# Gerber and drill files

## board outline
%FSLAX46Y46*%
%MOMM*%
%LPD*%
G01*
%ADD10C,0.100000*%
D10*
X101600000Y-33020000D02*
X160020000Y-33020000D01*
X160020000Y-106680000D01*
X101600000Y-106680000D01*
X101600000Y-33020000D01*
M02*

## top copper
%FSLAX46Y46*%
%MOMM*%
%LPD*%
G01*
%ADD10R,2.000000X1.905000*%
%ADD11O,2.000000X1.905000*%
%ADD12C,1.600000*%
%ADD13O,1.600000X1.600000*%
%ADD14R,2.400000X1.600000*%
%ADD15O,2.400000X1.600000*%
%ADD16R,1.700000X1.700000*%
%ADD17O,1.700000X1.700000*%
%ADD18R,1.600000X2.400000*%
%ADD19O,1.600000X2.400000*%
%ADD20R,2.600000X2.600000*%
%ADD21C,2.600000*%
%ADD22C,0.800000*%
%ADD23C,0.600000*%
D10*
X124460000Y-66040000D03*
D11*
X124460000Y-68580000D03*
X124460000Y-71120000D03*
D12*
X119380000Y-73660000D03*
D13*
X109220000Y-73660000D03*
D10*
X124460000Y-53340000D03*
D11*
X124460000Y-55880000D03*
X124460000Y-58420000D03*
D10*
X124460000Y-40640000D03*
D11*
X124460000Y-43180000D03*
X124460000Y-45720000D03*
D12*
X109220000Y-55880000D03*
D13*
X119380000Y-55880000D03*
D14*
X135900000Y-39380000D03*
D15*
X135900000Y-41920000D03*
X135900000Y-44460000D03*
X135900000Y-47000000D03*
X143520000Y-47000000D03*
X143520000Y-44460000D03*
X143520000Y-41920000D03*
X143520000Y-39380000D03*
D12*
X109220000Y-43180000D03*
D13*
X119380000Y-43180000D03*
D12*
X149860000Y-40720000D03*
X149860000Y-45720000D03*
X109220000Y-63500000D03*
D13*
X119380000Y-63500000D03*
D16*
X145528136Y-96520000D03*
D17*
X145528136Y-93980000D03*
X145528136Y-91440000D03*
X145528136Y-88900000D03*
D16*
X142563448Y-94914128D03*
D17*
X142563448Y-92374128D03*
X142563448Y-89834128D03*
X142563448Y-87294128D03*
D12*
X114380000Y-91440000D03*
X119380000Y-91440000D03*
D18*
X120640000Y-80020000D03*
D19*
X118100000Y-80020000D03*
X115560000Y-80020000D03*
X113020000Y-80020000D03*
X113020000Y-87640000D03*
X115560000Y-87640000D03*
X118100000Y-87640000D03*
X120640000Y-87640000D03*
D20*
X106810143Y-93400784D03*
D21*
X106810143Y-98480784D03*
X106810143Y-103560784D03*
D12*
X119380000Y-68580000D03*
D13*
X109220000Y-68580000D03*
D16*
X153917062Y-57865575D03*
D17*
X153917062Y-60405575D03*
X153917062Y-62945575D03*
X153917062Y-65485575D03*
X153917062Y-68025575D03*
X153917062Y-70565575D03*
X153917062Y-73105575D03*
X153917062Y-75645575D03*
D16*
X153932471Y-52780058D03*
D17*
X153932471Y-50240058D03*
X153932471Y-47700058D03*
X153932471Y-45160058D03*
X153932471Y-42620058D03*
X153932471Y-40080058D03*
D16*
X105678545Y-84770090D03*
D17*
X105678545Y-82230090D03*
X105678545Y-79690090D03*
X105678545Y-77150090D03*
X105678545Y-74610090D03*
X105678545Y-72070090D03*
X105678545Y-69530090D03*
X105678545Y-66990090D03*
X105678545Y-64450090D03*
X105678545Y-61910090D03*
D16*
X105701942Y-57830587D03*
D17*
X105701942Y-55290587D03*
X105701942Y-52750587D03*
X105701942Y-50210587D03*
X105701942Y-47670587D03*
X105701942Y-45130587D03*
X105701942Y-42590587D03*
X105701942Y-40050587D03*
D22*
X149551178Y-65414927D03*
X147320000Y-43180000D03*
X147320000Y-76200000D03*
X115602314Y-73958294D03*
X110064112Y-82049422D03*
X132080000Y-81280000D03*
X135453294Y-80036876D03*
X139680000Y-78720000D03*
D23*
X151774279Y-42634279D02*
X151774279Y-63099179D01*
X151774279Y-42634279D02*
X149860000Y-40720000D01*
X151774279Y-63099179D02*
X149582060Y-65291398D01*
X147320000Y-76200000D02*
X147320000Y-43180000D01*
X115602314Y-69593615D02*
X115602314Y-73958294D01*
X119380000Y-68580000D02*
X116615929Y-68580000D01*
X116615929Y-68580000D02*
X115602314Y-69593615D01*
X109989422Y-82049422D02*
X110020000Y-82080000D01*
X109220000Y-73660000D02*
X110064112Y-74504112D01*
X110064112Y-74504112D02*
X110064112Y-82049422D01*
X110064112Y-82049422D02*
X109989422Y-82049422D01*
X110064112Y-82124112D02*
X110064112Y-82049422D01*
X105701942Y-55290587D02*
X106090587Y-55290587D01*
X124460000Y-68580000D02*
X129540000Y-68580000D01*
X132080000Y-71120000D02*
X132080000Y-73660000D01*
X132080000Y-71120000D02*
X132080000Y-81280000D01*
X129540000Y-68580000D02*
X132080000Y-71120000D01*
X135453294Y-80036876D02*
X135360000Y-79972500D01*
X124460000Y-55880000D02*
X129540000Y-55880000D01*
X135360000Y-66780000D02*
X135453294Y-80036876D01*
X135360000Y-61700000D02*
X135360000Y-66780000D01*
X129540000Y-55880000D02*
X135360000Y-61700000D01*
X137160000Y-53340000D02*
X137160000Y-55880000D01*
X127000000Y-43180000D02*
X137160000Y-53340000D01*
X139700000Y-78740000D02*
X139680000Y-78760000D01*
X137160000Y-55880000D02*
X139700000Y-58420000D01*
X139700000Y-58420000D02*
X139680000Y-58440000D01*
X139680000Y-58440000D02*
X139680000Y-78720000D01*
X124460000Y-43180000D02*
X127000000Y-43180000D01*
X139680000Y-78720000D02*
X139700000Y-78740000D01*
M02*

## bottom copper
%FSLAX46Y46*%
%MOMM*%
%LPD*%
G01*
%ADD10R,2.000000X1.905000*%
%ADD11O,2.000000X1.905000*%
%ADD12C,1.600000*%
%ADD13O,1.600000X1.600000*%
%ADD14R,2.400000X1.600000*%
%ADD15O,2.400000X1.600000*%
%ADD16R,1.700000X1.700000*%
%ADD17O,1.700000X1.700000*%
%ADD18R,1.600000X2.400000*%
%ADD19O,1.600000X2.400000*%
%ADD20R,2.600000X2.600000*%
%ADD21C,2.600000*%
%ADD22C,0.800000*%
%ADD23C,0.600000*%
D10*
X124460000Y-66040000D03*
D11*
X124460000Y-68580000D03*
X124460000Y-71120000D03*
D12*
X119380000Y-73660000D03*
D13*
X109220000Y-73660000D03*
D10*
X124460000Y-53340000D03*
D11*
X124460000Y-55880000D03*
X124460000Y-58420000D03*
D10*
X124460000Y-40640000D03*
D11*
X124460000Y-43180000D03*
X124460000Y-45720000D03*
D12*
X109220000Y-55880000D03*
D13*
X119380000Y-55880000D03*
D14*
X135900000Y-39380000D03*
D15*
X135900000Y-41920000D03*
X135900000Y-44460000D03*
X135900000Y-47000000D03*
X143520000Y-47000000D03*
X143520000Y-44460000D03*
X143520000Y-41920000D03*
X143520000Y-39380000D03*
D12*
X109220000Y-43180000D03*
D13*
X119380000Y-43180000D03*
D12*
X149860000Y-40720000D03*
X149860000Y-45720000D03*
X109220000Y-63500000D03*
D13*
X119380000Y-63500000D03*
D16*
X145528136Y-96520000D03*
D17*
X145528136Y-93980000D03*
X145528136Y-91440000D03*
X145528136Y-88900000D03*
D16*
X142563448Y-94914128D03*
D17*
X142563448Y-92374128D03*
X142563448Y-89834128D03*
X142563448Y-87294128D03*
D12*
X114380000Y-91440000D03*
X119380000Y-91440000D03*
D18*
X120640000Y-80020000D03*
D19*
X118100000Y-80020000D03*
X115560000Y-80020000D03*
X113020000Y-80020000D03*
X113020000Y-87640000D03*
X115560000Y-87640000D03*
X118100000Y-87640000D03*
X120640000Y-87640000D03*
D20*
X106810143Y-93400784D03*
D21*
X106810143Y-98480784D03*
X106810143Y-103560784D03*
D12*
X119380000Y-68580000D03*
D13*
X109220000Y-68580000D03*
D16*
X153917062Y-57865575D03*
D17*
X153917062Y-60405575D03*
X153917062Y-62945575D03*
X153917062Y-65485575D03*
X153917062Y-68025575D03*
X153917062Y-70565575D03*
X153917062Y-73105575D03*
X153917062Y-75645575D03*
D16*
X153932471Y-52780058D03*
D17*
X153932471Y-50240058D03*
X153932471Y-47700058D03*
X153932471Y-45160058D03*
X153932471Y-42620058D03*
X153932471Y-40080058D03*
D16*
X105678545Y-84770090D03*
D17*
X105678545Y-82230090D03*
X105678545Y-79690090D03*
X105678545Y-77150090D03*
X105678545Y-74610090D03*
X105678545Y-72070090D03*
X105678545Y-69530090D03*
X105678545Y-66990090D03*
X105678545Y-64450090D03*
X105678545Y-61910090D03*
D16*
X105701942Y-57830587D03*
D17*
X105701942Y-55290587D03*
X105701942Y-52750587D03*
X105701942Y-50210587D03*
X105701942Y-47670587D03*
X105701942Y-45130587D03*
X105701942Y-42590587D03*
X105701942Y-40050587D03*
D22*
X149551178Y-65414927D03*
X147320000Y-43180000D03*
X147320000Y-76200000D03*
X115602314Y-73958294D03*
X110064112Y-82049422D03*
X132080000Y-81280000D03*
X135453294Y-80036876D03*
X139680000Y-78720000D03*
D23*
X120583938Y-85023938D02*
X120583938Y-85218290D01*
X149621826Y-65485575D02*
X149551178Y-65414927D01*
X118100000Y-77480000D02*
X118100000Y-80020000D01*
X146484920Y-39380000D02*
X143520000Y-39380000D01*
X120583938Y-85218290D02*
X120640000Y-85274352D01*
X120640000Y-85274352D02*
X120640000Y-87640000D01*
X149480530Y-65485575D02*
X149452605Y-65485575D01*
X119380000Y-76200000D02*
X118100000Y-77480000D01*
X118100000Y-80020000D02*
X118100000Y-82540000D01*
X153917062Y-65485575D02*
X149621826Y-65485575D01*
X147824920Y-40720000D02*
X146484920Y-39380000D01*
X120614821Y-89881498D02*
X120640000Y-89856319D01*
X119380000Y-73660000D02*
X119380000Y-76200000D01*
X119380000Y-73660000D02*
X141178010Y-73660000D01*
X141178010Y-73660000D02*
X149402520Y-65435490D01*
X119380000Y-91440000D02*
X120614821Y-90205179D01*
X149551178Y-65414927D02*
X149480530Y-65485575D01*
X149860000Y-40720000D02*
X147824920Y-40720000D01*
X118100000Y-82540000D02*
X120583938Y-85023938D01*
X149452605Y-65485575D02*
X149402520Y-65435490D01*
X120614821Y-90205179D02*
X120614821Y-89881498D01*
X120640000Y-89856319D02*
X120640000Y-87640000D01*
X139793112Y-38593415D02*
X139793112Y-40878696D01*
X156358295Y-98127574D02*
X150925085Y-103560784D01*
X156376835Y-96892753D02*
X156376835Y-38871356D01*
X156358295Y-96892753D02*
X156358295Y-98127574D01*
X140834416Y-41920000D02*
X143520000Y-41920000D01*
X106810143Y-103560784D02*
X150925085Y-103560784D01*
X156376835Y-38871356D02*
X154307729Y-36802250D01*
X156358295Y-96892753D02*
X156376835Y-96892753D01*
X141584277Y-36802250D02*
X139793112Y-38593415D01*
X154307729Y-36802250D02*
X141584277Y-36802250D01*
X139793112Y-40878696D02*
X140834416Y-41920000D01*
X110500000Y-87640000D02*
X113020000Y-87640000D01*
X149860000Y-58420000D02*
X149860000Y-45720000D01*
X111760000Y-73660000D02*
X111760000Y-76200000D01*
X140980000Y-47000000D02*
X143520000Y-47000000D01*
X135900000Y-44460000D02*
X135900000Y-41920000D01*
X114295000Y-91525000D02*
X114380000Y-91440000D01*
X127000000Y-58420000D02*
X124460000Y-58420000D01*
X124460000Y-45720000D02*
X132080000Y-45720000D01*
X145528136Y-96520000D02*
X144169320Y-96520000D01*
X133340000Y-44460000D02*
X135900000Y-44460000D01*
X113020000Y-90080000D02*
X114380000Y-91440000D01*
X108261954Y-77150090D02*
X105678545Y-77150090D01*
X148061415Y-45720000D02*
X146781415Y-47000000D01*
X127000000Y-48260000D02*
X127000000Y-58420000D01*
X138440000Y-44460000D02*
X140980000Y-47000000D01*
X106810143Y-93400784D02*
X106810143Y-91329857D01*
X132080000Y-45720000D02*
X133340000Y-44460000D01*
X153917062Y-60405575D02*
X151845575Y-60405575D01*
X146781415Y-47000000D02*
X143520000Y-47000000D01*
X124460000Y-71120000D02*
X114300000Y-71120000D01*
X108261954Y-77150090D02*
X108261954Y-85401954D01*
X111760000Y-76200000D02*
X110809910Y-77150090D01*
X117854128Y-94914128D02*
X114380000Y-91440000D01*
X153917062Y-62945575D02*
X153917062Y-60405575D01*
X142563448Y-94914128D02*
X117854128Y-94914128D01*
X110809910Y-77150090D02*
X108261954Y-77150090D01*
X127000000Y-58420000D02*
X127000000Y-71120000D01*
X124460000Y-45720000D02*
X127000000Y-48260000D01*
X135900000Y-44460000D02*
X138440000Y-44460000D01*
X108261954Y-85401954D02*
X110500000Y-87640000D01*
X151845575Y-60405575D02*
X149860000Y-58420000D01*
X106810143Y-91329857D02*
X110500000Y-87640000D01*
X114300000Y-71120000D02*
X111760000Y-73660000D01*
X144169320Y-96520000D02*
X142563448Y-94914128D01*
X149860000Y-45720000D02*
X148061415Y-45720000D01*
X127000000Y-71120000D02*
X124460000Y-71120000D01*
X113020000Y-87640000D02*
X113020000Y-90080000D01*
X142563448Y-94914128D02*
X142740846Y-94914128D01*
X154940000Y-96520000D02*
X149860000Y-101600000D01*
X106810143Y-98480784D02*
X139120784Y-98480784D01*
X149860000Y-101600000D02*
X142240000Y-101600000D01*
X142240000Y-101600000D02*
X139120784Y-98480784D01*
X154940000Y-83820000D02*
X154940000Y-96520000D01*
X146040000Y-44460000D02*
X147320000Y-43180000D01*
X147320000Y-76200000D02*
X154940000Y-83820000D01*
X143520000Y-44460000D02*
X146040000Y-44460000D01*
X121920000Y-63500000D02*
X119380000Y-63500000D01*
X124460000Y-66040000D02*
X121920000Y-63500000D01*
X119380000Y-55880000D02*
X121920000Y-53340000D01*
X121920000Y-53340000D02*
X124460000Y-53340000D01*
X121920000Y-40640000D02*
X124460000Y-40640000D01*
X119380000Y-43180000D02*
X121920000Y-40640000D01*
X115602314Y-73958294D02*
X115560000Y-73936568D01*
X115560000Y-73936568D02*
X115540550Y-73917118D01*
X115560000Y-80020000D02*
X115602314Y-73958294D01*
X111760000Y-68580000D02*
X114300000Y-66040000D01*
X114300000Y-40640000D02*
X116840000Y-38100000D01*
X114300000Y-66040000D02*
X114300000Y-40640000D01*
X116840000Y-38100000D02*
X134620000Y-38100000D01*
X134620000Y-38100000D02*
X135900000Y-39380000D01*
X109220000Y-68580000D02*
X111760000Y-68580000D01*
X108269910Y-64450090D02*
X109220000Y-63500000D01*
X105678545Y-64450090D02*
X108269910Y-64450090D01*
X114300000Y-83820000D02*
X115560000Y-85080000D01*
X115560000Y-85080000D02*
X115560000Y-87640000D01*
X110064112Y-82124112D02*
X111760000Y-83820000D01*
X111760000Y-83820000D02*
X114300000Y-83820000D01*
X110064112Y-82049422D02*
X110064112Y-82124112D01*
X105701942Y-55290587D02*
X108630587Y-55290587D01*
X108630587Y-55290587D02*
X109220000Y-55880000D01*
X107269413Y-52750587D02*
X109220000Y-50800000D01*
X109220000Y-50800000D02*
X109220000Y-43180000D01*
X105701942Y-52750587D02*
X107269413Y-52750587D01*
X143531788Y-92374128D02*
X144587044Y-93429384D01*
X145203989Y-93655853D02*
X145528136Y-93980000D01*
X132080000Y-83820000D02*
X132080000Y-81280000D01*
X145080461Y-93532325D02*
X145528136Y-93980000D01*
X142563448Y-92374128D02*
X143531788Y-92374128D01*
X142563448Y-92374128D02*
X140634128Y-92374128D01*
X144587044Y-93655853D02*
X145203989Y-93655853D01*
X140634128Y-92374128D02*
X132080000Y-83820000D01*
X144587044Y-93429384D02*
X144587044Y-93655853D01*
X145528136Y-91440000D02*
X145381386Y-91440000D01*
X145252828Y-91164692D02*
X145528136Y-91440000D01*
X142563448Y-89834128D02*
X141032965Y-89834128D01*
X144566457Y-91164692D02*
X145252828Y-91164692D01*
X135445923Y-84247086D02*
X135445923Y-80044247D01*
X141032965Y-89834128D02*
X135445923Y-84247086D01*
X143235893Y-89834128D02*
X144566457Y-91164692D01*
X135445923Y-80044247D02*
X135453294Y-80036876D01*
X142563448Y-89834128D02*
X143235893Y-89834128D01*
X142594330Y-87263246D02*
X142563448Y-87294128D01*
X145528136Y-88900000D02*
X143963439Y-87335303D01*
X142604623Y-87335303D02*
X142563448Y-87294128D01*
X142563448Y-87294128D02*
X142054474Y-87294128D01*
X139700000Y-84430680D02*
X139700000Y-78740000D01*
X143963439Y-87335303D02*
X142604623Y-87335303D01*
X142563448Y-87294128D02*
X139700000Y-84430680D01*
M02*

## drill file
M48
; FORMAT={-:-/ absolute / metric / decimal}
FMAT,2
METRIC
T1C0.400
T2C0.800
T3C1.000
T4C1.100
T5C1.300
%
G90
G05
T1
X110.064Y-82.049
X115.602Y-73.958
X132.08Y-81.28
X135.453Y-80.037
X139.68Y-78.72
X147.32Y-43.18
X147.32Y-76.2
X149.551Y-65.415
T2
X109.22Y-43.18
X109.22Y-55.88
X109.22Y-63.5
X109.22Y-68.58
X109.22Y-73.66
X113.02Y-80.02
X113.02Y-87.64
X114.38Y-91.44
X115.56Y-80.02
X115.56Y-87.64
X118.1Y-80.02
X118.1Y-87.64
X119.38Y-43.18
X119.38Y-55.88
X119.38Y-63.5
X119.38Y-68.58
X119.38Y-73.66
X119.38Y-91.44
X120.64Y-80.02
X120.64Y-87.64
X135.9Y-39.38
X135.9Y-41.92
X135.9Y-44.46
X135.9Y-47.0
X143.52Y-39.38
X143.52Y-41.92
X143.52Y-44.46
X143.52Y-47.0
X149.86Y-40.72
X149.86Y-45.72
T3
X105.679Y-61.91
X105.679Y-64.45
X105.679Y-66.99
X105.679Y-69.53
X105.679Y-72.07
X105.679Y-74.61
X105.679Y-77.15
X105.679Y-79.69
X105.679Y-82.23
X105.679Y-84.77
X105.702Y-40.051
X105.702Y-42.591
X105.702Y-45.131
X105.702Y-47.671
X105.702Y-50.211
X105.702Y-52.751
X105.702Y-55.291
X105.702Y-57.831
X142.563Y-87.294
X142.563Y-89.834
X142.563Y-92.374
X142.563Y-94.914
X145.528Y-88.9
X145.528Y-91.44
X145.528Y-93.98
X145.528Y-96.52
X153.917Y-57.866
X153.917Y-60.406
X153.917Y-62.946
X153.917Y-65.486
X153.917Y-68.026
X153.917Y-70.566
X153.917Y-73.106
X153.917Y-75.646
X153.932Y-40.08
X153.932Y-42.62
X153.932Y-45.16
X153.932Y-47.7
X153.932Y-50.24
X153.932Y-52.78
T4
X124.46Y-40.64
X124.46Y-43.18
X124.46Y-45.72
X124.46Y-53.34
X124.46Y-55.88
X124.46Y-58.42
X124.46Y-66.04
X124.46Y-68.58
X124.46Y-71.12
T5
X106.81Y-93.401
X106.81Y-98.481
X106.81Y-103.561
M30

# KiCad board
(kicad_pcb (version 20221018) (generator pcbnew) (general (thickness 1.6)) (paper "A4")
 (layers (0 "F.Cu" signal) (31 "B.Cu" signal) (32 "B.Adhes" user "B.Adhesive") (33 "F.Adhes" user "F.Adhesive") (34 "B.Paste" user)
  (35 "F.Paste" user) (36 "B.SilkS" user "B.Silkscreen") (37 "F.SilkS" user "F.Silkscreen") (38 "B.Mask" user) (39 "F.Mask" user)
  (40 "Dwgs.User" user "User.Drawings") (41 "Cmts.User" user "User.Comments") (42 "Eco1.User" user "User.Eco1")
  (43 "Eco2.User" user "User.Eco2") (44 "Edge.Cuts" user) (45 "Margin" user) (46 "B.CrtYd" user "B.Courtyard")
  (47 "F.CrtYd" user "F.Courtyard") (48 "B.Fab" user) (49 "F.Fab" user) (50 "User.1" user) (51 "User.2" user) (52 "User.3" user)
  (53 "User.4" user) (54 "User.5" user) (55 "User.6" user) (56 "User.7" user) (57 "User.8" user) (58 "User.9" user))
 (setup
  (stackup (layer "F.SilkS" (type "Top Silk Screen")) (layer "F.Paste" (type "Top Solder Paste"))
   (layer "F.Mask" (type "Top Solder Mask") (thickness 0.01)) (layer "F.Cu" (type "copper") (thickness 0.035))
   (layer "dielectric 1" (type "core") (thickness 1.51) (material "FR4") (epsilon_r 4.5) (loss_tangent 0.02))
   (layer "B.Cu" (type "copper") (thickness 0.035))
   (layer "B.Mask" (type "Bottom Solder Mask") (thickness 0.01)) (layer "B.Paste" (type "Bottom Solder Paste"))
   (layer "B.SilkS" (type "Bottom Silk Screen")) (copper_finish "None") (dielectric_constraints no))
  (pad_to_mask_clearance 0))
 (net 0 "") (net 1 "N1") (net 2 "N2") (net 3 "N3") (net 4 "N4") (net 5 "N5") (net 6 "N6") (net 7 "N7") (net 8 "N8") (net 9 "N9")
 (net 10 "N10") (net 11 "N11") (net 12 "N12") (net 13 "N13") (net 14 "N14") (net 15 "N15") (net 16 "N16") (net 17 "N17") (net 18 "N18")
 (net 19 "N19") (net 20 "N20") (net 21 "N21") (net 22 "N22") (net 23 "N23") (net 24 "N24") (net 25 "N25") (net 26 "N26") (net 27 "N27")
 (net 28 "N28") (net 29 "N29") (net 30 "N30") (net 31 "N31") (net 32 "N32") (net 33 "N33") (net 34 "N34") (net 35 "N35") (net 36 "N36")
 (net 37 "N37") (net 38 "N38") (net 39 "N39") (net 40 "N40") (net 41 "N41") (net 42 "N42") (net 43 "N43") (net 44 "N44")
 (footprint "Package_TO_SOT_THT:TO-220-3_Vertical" (layer "F.Cu") (at 124.46 66.04 -90)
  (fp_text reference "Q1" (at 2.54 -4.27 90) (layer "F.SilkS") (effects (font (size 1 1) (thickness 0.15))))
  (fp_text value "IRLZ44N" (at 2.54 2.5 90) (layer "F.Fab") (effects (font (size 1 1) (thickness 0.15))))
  (pad "1" thru_hole rect (at 0 0 270) (size 1.905 2) (drill 1.1) (layers "*.Cu" "*.Mask") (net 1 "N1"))
  (pad "2" thru_hole oval (at 2.54 0 270) (size 1.905 2) (drill 1.1) (layers "*.Cu" "*.Mask") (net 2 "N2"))
  (pad "3" thru_hole oval (at 5.08 0 270) (size 1.905 2) (drill 1.1) (layers "*.Cu" "*.Mask") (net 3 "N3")))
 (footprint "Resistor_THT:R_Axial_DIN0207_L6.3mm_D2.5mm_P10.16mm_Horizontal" (layer "F.Cu") (at 119.38 73.66 180)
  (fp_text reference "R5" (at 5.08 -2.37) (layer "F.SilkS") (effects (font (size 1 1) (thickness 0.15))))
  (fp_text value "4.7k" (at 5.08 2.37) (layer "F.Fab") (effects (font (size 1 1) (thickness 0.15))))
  (pad "1" thru_hole circle (at 0 0 180) (size 1.6 1.6) (drill 0.8) (layers "*.Cu" "*.Mask") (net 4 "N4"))
  (pad "2" thru_hole oval (at 10.16 0 180) (size 1.6 1.6) (drill 0.8) (layers "*.Cu" "*.Mask") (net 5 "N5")))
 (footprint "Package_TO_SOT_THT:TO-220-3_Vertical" (layer "F.Cu") (at 124.46 53.34 -90)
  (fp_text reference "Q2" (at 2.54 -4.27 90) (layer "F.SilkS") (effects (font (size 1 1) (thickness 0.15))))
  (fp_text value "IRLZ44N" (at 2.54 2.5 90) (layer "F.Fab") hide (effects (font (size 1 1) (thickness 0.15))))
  (pad "1" thru_hole rect (at 0 0 270) (size 1.905 2) (drill 1.1) (layers "*.Cu" "*.Mask") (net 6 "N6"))
  (pad "2" thru_hole oval (at 2.54 0 270) (size 1.905 2) (drill 1.1) (layers "*.Cu" "*.Mask") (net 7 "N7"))
  (pad "3" thru_hole oval (at 5.08 0 270) (size 1.905 2) (drill 1.1) (layers "*.Cu" "*.Mask") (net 3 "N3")))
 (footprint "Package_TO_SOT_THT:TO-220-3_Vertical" (layer "F.Cu") (at 124.46 40.64 -90)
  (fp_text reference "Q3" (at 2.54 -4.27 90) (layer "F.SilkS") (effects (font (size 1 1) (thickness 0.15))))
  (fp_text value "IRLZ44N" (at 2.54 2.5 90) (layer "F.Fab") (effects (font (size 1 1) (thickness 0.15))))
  (pad "1" thru_hole rect (at 0 0 270) (size 1.905 2) (drill 1.1) (layers "*.Cu" "*.Mask") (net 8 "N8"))
  (pad "2" thru_hole oval (at 2.54 0 270) (size 1.905 2) (drill 1.1) (layers "*.Cu" "*.Mask") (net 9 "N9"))
  (pad "3" thru_hole oval (at 5.08 0 270) (size 1.905 2) (drill 1.1) (layers "*.Cu" "*.Mask") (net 3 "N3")))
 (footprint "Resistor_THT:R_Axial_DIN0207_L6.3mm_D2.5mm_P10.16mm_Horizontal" (layer "F.Cu") (at 109.22 55.88)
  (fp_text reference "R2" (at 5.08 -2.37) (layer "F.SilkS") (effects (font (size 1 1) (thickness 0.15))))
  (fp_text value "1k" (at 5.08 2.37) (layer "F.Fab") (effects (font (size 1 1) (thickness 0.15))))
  (pad "1" thru_hole circle (at 0 0) (size 1.6 1.6) (drill 0.8) (layers "*.Cu" "*.Mask") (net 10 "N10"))
  (pad "2" thru_hole oval (at 10.16 0) (size 1.6 1.6) (drill 0.8) (layers "*.Cu" "*.Mask") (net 6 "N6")))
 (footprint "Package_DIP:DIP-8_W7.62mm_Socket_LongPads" (layer "F.Cu") (at 135.9 39.38)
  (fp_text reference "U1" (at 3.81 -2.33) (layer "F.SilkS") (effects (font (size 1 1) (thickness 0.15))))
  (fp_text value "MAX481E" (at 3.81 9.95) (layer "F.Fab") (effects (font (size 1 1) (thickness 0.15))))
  (pad "1" thru_hole rect (at 0 0) (size 2.4 1.6) (drill 0.8) (layers "*.Cu" "*.Mask") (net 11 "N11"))
  (pad "2" thru_hole oval (at 0 2.54) (size 2.4 1.6) (drill 0.8) (layers "*.Cu" "*.Mask") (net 3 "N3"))
  (pad "3" thru_hole oval (at 0 5.08) (size 2.4 1.6) (drill 0.8) (layers "*.Cu" "*.Mask") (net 3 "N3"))
  (pad "4" thru_hole oval (at 0 7.62) (size 2.4 1.6) (drill 0.8) (layers "*.Cu" "*.Mask") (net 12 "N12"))
  (pad "5" thru_hole oval (at 7.62 7.62) (size 2.4 1.6) (drill 0.8) (layers "*.Cu" "*.Mask") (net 3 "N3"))
  (pad "6" thru_hole oval (at 7.62 5.08) (size 2.4 1.6) (drill 0.8) (layers "*.Cu" "*.Mask") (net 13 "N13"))
  (pad "7" thru_hole oval (at 7.62 2.54) (size 2.4 1.6) (drill 0.8) (layers "*.Cu" "*.Mask") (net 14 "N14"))
  (pad "8" thru_hole oval (at 7.62 0) (size 2.4 1.6) (drill 0.8) (layers "*.Cu" "*.Mask") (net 4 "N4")))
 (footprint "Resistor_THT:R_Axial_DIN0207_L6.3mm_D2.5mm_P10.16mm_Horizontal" (layer "F.Cu") (at 109.22 43.18)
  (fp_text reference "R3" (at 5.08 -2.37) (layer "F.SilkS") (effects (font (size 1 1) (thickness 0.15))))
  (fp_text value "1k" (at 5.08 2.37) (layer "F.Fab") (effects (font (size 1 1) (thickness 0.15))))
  (pad "1" thru_hole circle (at 0 0) (size 1.6 1.6) (drill 0.8) (layers "*.Cu" "*.Mask") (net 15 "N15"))
  (pad "2" thru_hole oval (at 10.16 0) (size 1.6 1.6) (drill 0.8) (layers "*.Cu" "*.Mask") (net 8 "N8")))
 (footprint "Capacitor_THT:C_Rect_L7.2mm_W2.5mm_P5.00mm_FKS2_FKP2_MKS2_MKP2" (layer "F.Cu") (at 149.86 40.72 -90)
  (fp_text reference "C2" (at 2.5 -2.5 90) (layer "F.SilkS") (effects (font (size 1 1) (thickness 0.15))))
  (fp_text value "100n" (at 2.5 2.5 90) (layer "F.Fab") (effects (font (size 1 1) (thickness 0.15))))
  (pad "1" thru_hole circle (at 0 0 270) (size 1.6 1.6) (drill 0.8) (layers "*.Cu" "*.Mask") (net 4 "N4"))
  (pad "2" thru_hole circle (at 5 0 270) (size 1.6 1.6) (drill 0.8) (layers "*.Cu" "*.Mask") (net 3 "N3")))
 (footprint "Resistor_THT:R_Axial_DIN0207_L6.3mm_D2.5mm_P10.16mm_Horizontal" (layer "F.Cu") (at 109.22 63.5)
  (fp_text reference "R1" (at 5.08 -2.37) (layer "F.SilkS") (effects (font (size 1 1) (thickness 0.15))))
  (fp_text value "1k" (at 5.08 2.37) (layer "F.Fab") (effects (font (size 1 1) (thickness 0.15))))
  (pad "1" thru_hole circle (at 0 0) (size 1.6 1.6) (drill 0.8) (layers "*.Cu" "*.Mask") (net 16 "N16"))
  (pad "2" thru_hole oval (at 10.16 0) (size 1.6 1.6) (drill 0.8) (layers "*.Cu" "*.Mask") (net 1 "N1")))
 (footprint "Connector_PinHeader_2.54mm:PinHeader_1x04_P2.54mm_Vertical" (layer "F.Cu") (at 145.528136 96.52 180)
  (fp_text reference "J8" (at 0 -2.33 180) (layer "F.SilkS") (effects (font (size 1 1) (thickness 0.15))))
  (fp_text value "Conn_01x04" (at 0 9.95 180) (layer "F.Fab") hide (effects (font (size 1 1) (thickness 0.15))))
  (pad "1" thru_hole rect (at 0 0 180) (size 1.7 1.7) (drill 1) (layers "*.Cu" "*.Mask") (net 3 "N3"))
  (pad "2" thru_hole oval (at 0 2.54 180) (size 1.7 1.7) (drill 1) (layers "*.Cu" "*.Mask") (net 2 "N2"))
  (pad "3" thru_hole oval (at 0 5.08 180) (size 1.7 1.7) (drill 1) (layers "*.Cu" "*.Mask") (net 7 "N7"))
  (pad "4" thru_hole oval (at 0 7.62 180) (size 1.7 1.7) (drill 1) (layers "*.Cu" "*.Mask") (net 9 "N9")))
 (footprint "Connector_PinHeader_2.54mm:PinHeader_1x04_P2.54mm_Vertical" (layer "F.Cu") (at 142.563448 94.914128 180)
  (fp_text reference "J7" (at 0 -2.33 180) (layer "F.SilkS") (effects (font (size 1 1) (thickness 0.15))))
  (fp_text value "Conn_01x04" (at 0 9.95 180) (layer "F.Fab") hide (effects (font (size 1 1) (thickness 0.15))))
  (pad "1" thru_hole rect (at 0 0 180) (size 1.7 1.7) (drill 1) (layers "*.Cu" "*.Mask") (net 3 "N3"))
  (pad "2" thru_hole oval (at 0 2.54 180) (size 1.7 1.7) (drill 1) (layers "*.Cu" "*.Mask") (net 2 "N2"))
  (pad "3" thru_hole oval (at 0 5.08 180) (size 1.7 1.7) (drill 1) (layers "*.Cu" "*.Mask") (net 7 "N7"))
  (pad "4" thru_hole oval (at 0 7.62 180) (size 1.7 1.7) (drill 1) (layers "*.Cu" "*.Mask") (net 9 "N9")))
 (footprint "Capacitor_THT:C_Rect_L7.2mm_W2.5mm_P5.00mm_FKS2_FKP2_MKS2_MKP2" (layer "F.Cu") (at 114.38 91.44)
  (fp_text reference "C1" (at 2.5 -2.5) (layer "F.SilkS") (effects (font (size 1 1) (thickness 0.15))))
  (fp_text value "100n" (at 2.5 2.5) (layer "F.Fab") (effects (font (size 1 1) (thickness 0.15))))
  (pad "1" thru_hole circle (at 0 0) (size 1.6 1.6) (drill 0.8) (layers "*.Cu" "*.Mask") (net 3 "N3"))
  (pad "2" thru_hole circle (at 5 0) (size 1.6 1.6) (drill 0.8) (layers "*.Cu" "*.Mask") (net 4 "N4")))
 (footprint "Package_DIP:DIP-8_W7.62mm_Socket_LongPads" (layer "F.Cu") (at 120.64 80.02 -90)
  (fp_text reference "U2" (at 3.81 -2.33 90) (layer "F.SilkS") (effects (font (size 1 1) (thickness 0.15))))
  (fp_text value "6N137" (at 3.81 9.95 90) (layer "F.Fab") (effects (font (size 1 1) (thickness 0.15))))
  (pad "1" thru_hole rect (at 0 0 270) (size 2.4 1.6) (drill 0.8) (layers "*.Cu" "*.Mask") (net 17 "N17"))
  (pad "2" thru_hole oval (at 0 2.54 270) (size 2.4 1.6) (drill 0.8) (layers "*.Cu" "*.Mask") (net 4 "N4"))
  (pad "3" thru_hole oval (at 0 5.08 270) (size 2.4 1.6) (drill 0.8) (layers "*.Cu" "*.Mask") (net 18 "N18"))
  (pad "4" thru_hole oval (at 0 7.62 270) (size 2.4 1.6) (drill 0.8) (layers "*.Cu" "*.Mask"))
  (pad "5" thru_hole oval (at 7.62 7.62 270) (size 2.4 1.6) (drill 0.8) (layers "*.Cu" "*.Mask") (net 3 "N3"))
  (pad "6" thru_hole oval (at 7.62 5.08 270) (size 2.4 1.6) (drill 0.8) (layers "*.Cu" "*.Mask") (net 5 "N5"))
  (pad "7" thru_hole oval (at 7.62 2.54 270) (size 2.4 1.6) (drill 0.8) (layers "*.Cu" "*.Mask") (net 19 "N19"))
  (pad "8" thru_hole oval (at 7.62 0 270) (size 2.4 1.6) (drill 0.8) (layers "*.Cu" "*.Mask") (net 4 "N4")))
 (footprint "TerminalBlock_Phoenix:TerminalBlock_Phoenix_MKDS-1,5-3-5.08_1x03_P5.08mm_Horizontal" (layer "F.Cu")
  (at 106.810143 93.400784 -90)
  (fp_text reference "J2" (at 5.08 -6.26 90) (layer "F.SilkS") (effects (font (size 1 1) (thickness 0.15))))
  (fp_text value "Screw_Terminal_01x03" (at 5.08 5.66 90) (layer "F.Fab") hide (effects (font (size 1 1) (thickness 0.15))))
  (pad "1" thru_hole rect (at 0 0 270) (size 2.6 2.6) (drill 1.3) (layers "*.Cu" "*.Mask") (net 3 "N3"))
  (pad "2" thru_hole circle (at 5.08 0 270) (size 2.6 2.6) (drill 1.3) (layers "*.Cu" "*.Mask") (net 13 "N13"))
  (pad "3" thru_hole circle (at 10.16 0 270) (size 2.6 2.6) (drill 1.3) (layers "*.Cu" "*.Mask") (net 14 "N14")))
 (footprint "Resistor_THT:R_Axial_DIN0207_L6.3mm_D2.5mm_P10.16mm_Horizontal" (layer "F.Cu") (at 119.38 68.58 180)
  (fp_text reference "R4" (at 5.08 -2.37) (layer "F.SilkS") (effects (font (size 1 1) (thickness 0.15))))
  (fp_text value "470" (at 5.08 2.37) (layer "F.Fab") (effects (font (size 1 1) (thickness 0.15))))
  (pad "1" thru_hole circle (at 0 0 180) (size 1.6 1.6) (drill 0.8) (layers "*.Cu" "*.Mask") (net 18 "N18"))
  (pad "2" thru_hole oval (at 10.16 0 180) (size 1.6 1.6) (drill 0.8) (layers "*.Cu" "*.Mask") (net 11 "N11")))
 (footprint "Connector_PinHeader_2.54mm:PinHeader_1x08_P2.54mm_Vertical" (layer "B.Cu") (at 153.917062 57.865575 180)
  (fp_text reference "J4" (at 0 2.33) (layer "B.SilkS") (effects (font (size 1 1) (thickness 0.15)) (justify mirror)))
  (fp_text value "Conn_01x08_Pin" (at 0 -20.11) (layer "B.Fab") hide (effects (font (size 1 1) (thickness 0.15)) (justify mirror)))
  (pad "1" thru_hole rect (at 0 0 180) (size 1.7 1.7) (drill 1) (layers "*.Cu" "*.Mask") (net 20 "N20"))
  (pad "2" thru_hole oval (at 0 -2.54 180) (size 1.7 1.7) (drill 1) (layers "*.Cu" "*.Mask") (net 3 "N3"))
  (pad "3" thru_hole oval (at 0 -5.08 180) (size 1.7 1.7) (drill 1) (layers "*.Cu" "*.Mask") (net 3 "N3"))
  (pad "4" thru_hole oval (at 0 -7.62 180) (size 1.7 1.7) (drill 1) (layers "*.Cu" "*.Mask") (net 4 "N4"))
  (pad "5" thru_hole oval (at 0 -10.16 180) (size 1.7 1.7) (drill 1) (layers "*.Cu" "*.Mask") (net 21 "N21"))
  (pad "6" thru_hole oval (at 0 -12.7 180) (size 1.7 1.7) (drill 1) (layers "*.Cu" "*.Mask") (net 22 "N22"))
  (pad "7" thru_hole oval (at 0 -15.24 180) (size 1.7 1.7) (drill 1) (layers "*.Cu" "*.Mask") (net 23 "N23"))
  (pad "8" thru_hole oval (at 0 -17.78 180) (size 1.7 1.7) (drill 1) (layers "*.Cu" "*.Mask") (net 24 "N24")))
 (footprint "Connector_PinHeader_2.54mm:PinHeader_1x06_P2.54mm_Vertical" (layer "B.Cu") (at 153.932471 52.780058)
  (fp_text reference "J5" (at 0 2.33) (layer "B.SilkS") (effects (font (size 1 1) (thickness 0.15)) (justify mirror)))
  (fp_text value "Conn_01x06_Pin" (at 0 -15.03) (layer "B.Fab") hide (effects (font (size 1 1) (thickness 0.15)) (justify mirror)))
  (pad "1" thru_hole rect (at 0 0) (size 1.7 1.7) (drill 1) (layers "*.Cu" "*.Mask") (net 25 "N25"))
  (pad "2" thru_hole oval (at 0 -2.54) (size 1.7 1.7) (drill 1) (layers "*.Cu" "*.Mask") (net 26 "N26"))
  (pad "3" thru_hole oval (at 0 -5.08) (size 1.7 1.7) (drill 1) (layers "*.Cu" "*.Mask") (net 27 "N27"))
  (pad "4" thru_hole oval (at 0 -7.62) (size 1.7 1.7) (drill 1) (layers "*.Cu" "*.Mask") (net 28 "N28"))
  (pad "5" thru_hole oval (at 0 -10.16) (size 1.7 1.7) (drill 1) (layers "*.Cu" "*.Mask") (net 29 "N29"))
  (pad "6" thru_hole oval (at 0 -12.7) (size 1.7 1.7) (drill 1) (layers "*.Cu" "*.Mask") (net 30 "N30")))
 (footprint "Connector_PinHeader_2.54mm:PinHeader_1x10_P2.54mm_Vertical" (layer "B.Cu") (at 105.678545 84.77009)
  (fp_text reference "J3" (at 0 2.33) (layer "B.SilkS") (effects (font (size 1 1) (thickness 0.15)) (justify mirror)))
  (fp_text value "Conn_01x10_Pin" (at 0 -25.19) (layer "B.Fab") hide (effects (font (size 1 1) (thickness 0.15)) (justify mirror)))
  (pad "1" thru_hole rect (at 0 0) (size 1.7 1.7) (drill 1) (layers "*.Cu" "*.Mask") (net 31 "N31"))
  (pad "2" thru_hole oval (at 0 -2.54) (size 1.7 1.7) (drill 1) (layers "*.Cu" "*.Mask") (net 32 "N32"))
  (pad "3" thru_hole oval (at 0 -5.08) (size 1.7 1.7) (drill 1) (layers "*.Cu" "*.Mask") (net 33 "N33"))
  (pad "4" thru_hole oval (at 0 -7.62) (size 1.7 1.7) (drill 1) (layers "*.Cu" "*.Mask") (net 3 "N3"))
  (pad "5" thru_hole oval (at 0 -10.16) (size 1.7 1.7) (drill 1) (layers "*.Cu" "*.Mask") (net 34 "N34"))
  (pad "6" thru_hole oval (at 0 -12.7) (size 1.7 1.7) (drill 1) (layers "*.Cu" "*.Mask") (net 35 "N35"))
  (pad "7" thru_hole oval (at 0 -15.24) (size 1.7 1.7) (drill 1) (layers "*.Cu" "*.Mask") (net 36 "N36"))
  (pad "8" thru_hole oval (at 0 -17.78) (size 1.7 1.7) (drill 1) (layers "*.Cu" "*.Mask") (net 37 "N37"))
  (pad "9" thru_hole oval (at 0 -20.32) (size 1.7 1.7) (drill 1) (layers "*.Cu" "*.Mask") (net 16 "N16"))
  (pad "10" thru_hole oval (at 0 -22.86) (size 1.7 1.7) (drill 1) (layers "*.Cu" "*.Mask") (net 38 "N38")))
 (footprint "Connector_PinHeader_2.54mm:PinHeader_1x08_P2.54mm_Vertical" (layer "B.Cu") (at 105.701942 57.830587)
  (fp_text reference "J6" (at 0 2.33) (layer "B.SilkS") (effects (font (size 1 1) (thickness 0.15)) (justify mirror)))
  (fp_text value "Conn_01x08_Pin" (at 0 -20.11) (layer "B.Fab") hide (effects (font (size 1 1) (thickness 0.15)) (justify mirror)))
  (pad "1" thru_hole rect (at 0 0) (size 1.7 1.7) (drill 1) (layers "*.Cu" "*.Mask") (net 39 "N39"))
  (pad "2" thru_hole oval (at 0 -2.54) (size 1.7 1.7) (drill 1) (layers "*.Cu" "*.Mask") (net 10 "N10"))
  (pad "3" thru_hole oval (at 0 -5.08) (size 1.7 1.7) (drill 1) (layers "*.Cu" "*.Mask") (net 15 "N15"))
  (pad "4" thru_hole oval (at 0 -7.62) (size 1.7 1.7) (drill 1) (layers "*.Cu" "*.Mask") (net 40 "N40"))
  (pad "5" thru_hole oval (at 0 -10.16) (size 1.7 1.7) (drill 1) (layers "*.Cu" "*.Mask") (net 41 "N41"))
  (pad "6" thru_hole oval (at 0 -12.7) (size 1.7 1.7) (drill 1) (layers "*.Cu" "*.Mask") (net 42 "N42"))
  (pad "7" thru_hole oval (at 0 -15.24) (size 1.7 1.7) (drill 1) (layers "*.Cu" "*.Mask") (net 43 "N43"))
  (pad "8" thru_hole oval (at 0 -17.78) (size 1.7 1.7) (drill 1) (layers "*.Cu" "*.Mask") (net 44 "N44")))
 (gr_rect (start 101.6 33.02) (end 160.02 106.68) (stroke (width 0.1) (type default)) (fill none) (layer "Edge.Cuts"))
 (segment (start 151.774279 42.634279) (end 151.774279 63.099179) (width 0.6) (layer "F.Cu") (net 4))
 (segment (start 151.774279 42.634279) (end 149.86 40.72) (width 0.6) (layer "F.Cu") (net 4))
 (segment (start 151.774279 63.099179) (end 149.58206 65.291398) (width 0.6) (layer "F.Cu") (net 4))
 (via (at 149.551178 65.414927) (size 0.8) (drill 0.4) (layers "F.Cu" "B.Cu") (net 4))
 (segment (start 120.583938 85.023938) (end 120.583938 85.21829) (width 0.6) (layer "B.Cu") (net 4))
 (segment (start 149.621826 65.485575) (end 149.551178 65.414927) (width 0.6) (layer "B.Cu") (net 4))
 (segment (start 118.1 77.48) (end 118.1 80.02) (width 0.6) (layer "B.Cu") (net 4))
 (segment (start 146.48492 39.38) (end 143.52 39.38) (width 0.6) (layer "B.Cu") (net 4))
 (segment (start 120.583938 85.21829) (end 120.64 85.274352) (width 0.6) (layer "B.Cu") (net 4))
 (segment (start 120.64 85.274352) (end 120.64 87.64) (width 0.6) (layer "B.Cu") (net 4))
 (segment (start 149.48053 65.485575) (end 149.452605 65.485575) (width 0.6) (layer "B.Cu") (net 4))
 (segment (start 119.38 76.2) (end 118.1 77.48) (width 0.6) (layer "B.Cu") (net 4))
 (segment (start 118.1 80.02) (end 118.1 82.54) (width 0.6) (layer "B.Cu") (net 4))
 (segment (start 153.917062 65.485575) (end 149.621826 65.485575) (width 0.6) (layer "B.Cu") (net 4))
 (segment (start 147.82492 40.72) (end 146.48492 39.38) (width 0.6) (layer "B.Cu") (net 4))
 (segment (start 120.614821 89.881498) (end 120.64 89.856319) (width 0.6) (layer "B.Cu") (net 4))
 (segment (start 119.38 73.66) (end 119.38 76.2) (width 0.6) (layer "B.Cu") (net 4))
 (segment (start 119.38 73.66) (end 141.17801 73.66) (width 0.6) (layer "B.Cu") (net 4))
 (segment (start 141.17801 73.66) (end 149.40252 65.43549) (width 0.6) (layer "B.Cu") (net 4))
 (segment (start 119.38 91.44) (end 120.614821 90.205179) (width 0.6) (layer "B.Cu") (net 4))
 (segment (start 149.551178 65.414927) (end 149.48053 65.485575) (width 0.6) (layer "B.Cu") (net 4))
 (segment (start 149.86 40.72) (end 147.82492 40.72) (width 0.6) (layer "B.Cu") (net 4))
 (segment (start 118.1 82.54) (end 120.583938 85.023938) (width 0.6) (layer "B.Cu") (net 4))
 (segment (start 149.452605 65.485575) (end 149.40252 65.43549) (width 0.6) (layer "B.Cu") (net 4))
 (segment (start 120.614821 90.205179) (end 120.614821 89.881498) (width 0.6) (layer "B.Cu") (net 4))
 (segment (start 120.64 89.856319) (end 120.64 87.64) (width 0.6) (layer "B.Cu") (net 4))
 (segment (start 139.793112 38.593415) (end 139.793112 40.878696) (width 0.6) (layer "B.Cu") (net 14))
 (segment (start 156.358295 98.127574) (end 150.925085 103.560784) (width 0.6) (layer "B.Cu") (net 14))
 (segment (start 156.376835 96.892753) (end 156.376835 38.871356) (width 0.6) (layer "B.Cu") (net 14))
 (segment (start 156.358295 96.892753) (end 156.358295 98.127574) (width 0.6) (layer "B.Cu") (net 14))
 (segment (start 140.834416 41.92) (end 143.52 41.92) (width 0.6) (layer "B.Cu") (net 14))
 (segment (start 106.810143 103.560784) (end 150.925085 103.560784) (width 0.6) (layer "B.Cu") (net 14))
 (segment (start 156.376835 38.871356) (end 154.307729 36.80225) (width 0.6) (layer "B.Cu") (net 14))
 (segment (start 156.358295 96.892753) (end 156.376835 96.892753) (width 0.6) (layer "B.Cu") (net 14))
 (segment (start 141.584277 36.80225) (end 139.793112 38.593415) (width 0.6) (layer "B.Cu") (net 14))
 (segment (start 154.307729 36.80225) (end 141.584277 36.80225) (width 0.6) (layer "B.Cu") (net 14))
 (segment (start 139.793112 40.878696) (end 140.834416 41.92) (width 0.6) (layer "B.Cu") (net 14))
 (segment (start 110.5 87.64) (end 113.02 87.64) (width 0.6) (layer "B.Cu") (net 3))
 (segment (start 149.86 58.42) (end 149.86 45.72) (width 0.6) (layer "B.Cu") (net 3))
 (segment (start 111.76 73.66) (end 111.76 76.2) (width 0.6) (layer "B.Cu") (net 3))
 (segment (start 140.98 47) (end 143.52 47) (width 0.6) (layer "B.Cu") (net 3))
 (segment (start 135.9 44.46) (end 135.9 41.92) (width 0.6) (layer "B.Cu") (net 3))
 (segment (start 114.295 91.525) (end 114.38 91.44) (width 0.6) (layer "B.Cu") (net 3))
 (segment (start 127 58.42) (end 124.46 58.42) (width 0.6) (layer "B.Cu") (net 3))
 (segment (start 124.46 45.72) (end 132.08 45.72) (width 0.6) (layer "B.Cu") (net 3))
 (segment (start 145.528136 96.52) (end 144.16932 96.52) (width 0.6) (layer "B.Cu") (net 3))
 (segment (start 133.34 44.46) (end 135.9 44.46) (width 0.6) (layer "B.Cu") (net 3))
 (segment (start 113.02 90.08) (end 114.38 91.44) (width 0.6) (layer "B.Cu") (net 3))
 (segment (start 108.261954 77.15009) (end 105.678545 77.15009) (width 0.6) (layer "B.Cu") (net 3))
 (segment (start 148.061415 45.72) (end 146.781415 47) (width 0.6) (layer "B.Cu") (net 3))
 (segment (start 127 48.26) (end 127 58.42) (width 0.6) (layer "B.Cu") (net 3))
 (segment (start 138.44 44.46) (end 140.98 47) (width 0.6) (layer "B.Cu") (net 3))
 (segment (start 106.810143 93.400784) (end 106.810143 91.329857) (width 0.6) (layer "B.Cu") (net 3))
 (segment (start 132.08 45.72) (end 133.34 44.46) (width 0.6) (layer "B.Cu") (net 3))
 (segment (start 153.917062 60.405575) (end 151.845575 60.405575) (width 0.6) (layer "B.Cu") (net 3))
 (segment (start 146.781415 47) (end 143.52 47) (width 0.6) (layer "B.Cu") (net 3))
 (segment (start 124.46 71.12) (end 114.3 71.12) (width 0.6) (layer "B.Cu") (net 3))
 (segment (start 108.261954 77.15009) (end 108.261954 85.401954) (width 0.6) (layer "B.Cu") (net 3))
 (segment (start 111.76 76.2) (end 110.80991 77.15009) (width 0.6) (layer "B.Cu") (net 3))
 (segment (start 117.854128 94.914128) (end 114.38 91.44) (width 0.6) (layer "B.Cu") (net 3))
 (segment (start 153.917062 62.945575) (end 153.917062 60.405575) (width 0.6) (layer "B.Cu") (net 3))
 (segment (start 142.563448 94.914128) (end 117.854128 94.914128) (width 0.6) (layer "B.Cu") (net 3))
 (segment (start 110.80991 77.15009) (end 108.261954 77.15009) (width 0.6) (layer "B.Cu") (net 3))
 (segment (start 127 58.42) (end 127 71.12) (width 0.6) (layer "B.Cu") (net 3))
 (segment (start 124.46 45.72) (end 127 48.26) (width 0.6) (layer "B.Cu") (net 3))
 (segment (start 135.9 44.46) (end 138.44 44.46) (width 0.6) (layer "B.Cu") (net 3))
 (segment (start 108.261954 85.401954) (end 110.5 87.64) (width 0.6) (layer "B.Cu") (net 3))
 (segment (start 151.845575 60.405575) (end 149.86 58.42) (width 0.6) (layer "B.Cu") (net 3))
 (segment (start 106.810143 91.329857) (end 110.5 87.64) (width 0.6) (layer "B.Cu") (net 3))
 (segment (start 114.3 71.12) (end 111.76 73.66) (width 0.6) (layer "B.Cu") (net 3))
 (segment (start 144.16932 96.52) (end 142.563448 94.914128) (width 0.6) (layer "B.Cu") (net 3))
 (segment (start 149.86 45.72) (end 148.061415 45.72) (width 0.6) (layer "B.Cu") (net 3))
 (segment (start 127 71.12) (end 124.46 71.12) (width 0.6) (layer "B.Cu") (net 3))
 (segment (start 113.02 87.64) (end 113.02 90.08) (width 0.6) (layer "B.Cu") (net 3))
 (segment (start 142.563448 94.914128) (end 142.740846 94.914128) (width 0.6) (layer "B.Cu") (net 3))
 (segment (start 147.32 76.2) (end 147.32 43.18) (width 0.6) (layer "F.Cu") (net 13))
 (via (at 147.32 43.18) (size 0.8) (drill 0.4) (layers "F.Cu" "B.Cu") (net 13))
 (via (at 147.32 76.2) (size 0.8) (drill 0.4) (layers "F.Cu" "B.Cu") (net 13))
 (segment (start 154.94 96.52) (end 149.86 101.6) (width 0.6) (layer "B.Cu") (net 13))
 (segment (start 106.810143 98.480784) (end 139.120784 98.480784) (width 0.6) (layer "B.Cu") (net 13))
 (segment (start 149.86 101.6) (end 142.24 101.6) (width 0.6) (layer "B.Cu") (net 13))
 (segment (start 142.24 101.6) (end 139.120784 98.480784) (width 0.6) (layer "B.Cu") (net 13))
 (segment (start 154.94 83.82) (end 154.94 96.52) (width 0.6) (layer "B.Cu") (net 13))
 (segment (start 146.04 44.46) (end 147.32 43.18) (width 0.6) (layer "B.Cu") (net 13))
 (segment (start 147.32 76.2) (end 154.94 83.82) (width 0.6) (layer "B.Cu") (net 13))
 (segment (start 143.52 44.46) (end 146.04 44.46) (width 0.6) (layer "B.Cu") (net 13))
 (segment (start 121.92 63.5) (end 119.38 63.5) (width 0.6) (layer "B.Cu") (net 1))
 (segment (start 124.46 66.04) (end 121.92 63.5) (width 0.6) (layer "B.Cu") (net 1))
 (segment (start 119.38 55.88) (end 121.92 53.34) (width 0.6) (layer "B.Cu") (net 6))
 (segment (start 121.92 53.34) (end 124.46 53.34) (width 0.6) (layer "B.Cu") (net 6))
 (segment (start 121.92 40.64) (end 124.46 40.64) (width 0.6) (layer "B.Cu") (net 8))
 (segment (start 119.38 43.18) (end 121.92 40.64) (width 0.6) (layer "B.Cu") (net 8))
 (segment (start 115.602314 69.593615) (end 115.602314 73.958294) (width 0.6) (layer "F.Cu") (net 18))
 (segment (start 119.38 68.58) (end 116.615929 68.58) (width 0.6) (layer "F.Cu") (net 18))
 (segment (start 116.615929 68.58) (end 115.602314 69.593615) (width 0.6) (layer "F.Cu") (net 18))
 (via (at 115.602314 73.958294) (size 0.8) (drill 0.4) (layers "F.Cu" "B.Cu") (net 18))
 (segment (start 115.602314 73.958294) (end 115.56 73.936568) (width 0.6) (layer "B.Cu") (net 18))
 (segment (start 115.56 73.936568) (end 115.54055 73.917118) (width 0.6) (layer "B.Cu") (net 18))
 (segment (start 115.56 80.02) (end 115.602314 73.958294) (width 0.6) (layer "B.Cu") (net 18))
 (segment (start 111.76 68.58) (end 114.3 66.04) (width 0.6) (layer "B.Cu") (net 11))
 (segment (start 114.3 40.64) (end 116.84 38.1) (width 0.6) (layer "B.Cu") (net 11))
 (segment (start 114.3 66.04) (end 114.3 40.64) (width 0.6) (layer "B.Cu") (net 11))
 (segment (start 116.84 38.1) (end 134.62 38.1) (width 0.6) (layer "B.Cu") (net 11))
 (segment (start 134.62 38.1) (end 135.9 39.38) (width 0.6) (layer "B.Cu") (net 11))
 (segment (start 109.22 68.58) (end 111.76 68.58) (width 0.6) (layer "B.Cu") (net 11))
 (segment (start 108.26991 64.45009) (end 109.22 63.5) (width 0.6) (layer "B.Cu") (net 16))
 (segment (start 105.678545 64.45009) (end 108.26991 64.45009) (width 0.6) (layer "B.Cu") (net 16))
 (segment (start 109.989422 82.049422) (end 110.02 82.08) (width 0.6) (layer "F.Cu") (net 5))
 (segment (start 109.22 73.66) (end 110.064112 74.504112) (width 0.6) (layer "F.Cu") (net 5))
 (segment (start 110.064112 74.504112) (end 110.064112 82.049422) (width 0.6) (layer "F.Cu") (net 5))
 (segment (start 110.064112 82.049422) (end 109.989422 82.049422) (width 0.6) (layer "F.Cu") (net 5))
 (segment (start 110.064112 82.124112) (end 110.064112 82.049422) (width 0.6) (layer "F.Cu") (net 5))
 (via (at 110.064112 82.049422) (size 0.8) (drill 0.4) (layers "F.Cu" "B.Cu") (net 5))
 (segment (start 114.3 83.82) (end 115.56 85.08) (width 0.6) (layer "B.Cu") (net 5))
 (segment (start 115.56 85.08) (end 115.56 87.64) (width 0.6) (layer "B.Cu") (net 5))
 (segment (start 110.064112 82.124112) (end 111.76 83.82) (width 0.6) (layer "B.Cu") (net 5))
 (segment (start 111.76 83.82) (end 114.3 83.82) (width 0.6) (layer "B.Cu") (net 5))
 (segment (start 110.064112 82.049422) (end 110.064112 82.124112) (width 0.6) (layer "B.Cu") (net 5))
 (segment (start 105.701942 55.290587) (end 106.090587 55.290587) (width 0.6) (layer "F.Cu") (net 10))
 (segment (start 105.701942 55.290587) (end 108.630587 55.290587) (width 0.6) (layer "B.Cu") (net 10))
 (segment (start 108.630587 55.290587) (end 109.22 55.88) (width 0.6) (layer "B.Cu") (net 10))
 (segment (start 107.269413 52.750587) (end 109.22 50.8) (width 0.6) (layer "B.Cu") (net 15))
 (segment (start 109.22 50.8) (end 109.22 43.18) (width 0.6) (layer "B.Cu") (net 15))
 (segment (start 105.701942 52.750587) (end 107.269413 52.750587) (width 0.6) (layer "B.Cu") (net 15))
 (segment (start 124.46 68.58) (end 129.54 68.58) (width 0.6) (layer "F.Cu") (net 2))
 (segment (start 132.08 71.12) (end 132.08 73.66) (width 0.6) (layer "F.Cu") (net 2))
 (segment (start 132.08 71.12) (end 132.08 81.28) (width 0.6) (layer "F.Cu") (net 2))
 (segment (start 129.54 68.58) (end 132.08 71.12) (width 0.6) (layer "F.Cu") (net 2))
 (via (at 132.08 81.28) (size 0.8) (drill 0.4) (layers "F.Cu" "B.Cu") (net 2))
 (segment (start 143.531788 92.374128) (end 144.587044 93.429384) (width 0.6) (layer "B.Cu") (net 2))
 (segment (start 145.203989 93.655853) (end 145.528136 93.98) (width 0.6) (layer "B.Cu") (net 2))
 (segment (start 132.08 83.82) (end 132.08 81.28) (width 0.6) (layer "B.Cu") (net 2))
 (segment (start 145.080461 93.532325) (end 145.528136 93.98) (width 0.6) (layer "B.Cu") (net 2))
 (segment (start 142.563448 92.374128) (end 143.531788 92.374128) (width 0.6) (layer "B.Cu") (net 2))
 (segment (start 142.563448 92.374128) (end 140.634128 92.374128) (width 0.6) (layer "B.Cu") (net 2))
 (segment (start 144.587044 93.655853) (end 145.203989 93.655853) (width 0.6) (layer "B.Cu") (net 2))
 (segment (start 140.634128 92.374128) (end 132.08 83.82) (width 0.6) (layer "B.Cu") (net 2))
 (segment (start 144.587044 93.429384) (end 144.587044 93.655853) (width 0.6) (layer "B.Cu") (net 2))
 (segment (start 135.453294 80.036876) (end 135.36 79.9725) (width 0.6) (layer "F.Cu") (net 7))
 (segment (start 124.46 55.88) (end 129.54 55.88) (width 0.6) (layer "F.Cu") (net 7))
 (segment (start 135.36 66.78) (end 135.453294 80.036876) (width 0.6) (layer "F.Cu") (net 7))
 (segment (start 135.36 61.7) (end 135.36 66.78) (width 0.6) (layer "F.Cu") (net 7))
 (segment (start 129.54 55.88) (end 135.36 61.7) (width 0.6) (layer "F.Cu") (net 7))
 (via (at 135.453294 80.036876) (size 0.8) (drill 0.4) (layers "F.Cu" "B.Cu") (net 7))
 (segment (start 145.528136 91.44) (end 145.381386 91.44) (width 0.6) (layer "B.Cu") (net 7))
 (segment (start 145.252828 91.164692) (end 145.528136 91.44) (width 0.6) (layer "B.Cu") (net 7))
 (segment (start 142.563448 89.834128) (end 141.032965 89.834128) (width 0.6) (layer "B.Cu") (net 7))
 (segment (start 144.566457 91.164692) (end 145.252828 91.164692) (width 0.6) (layer "B.Cu") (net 7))
 (segment (start 135.445923 84.247086) (end 135.445923 80.044247) (width 0.6) (layer "B.Cu") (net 7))
 (segment (start 141.032965 89.834128) (end 135.445923 84.247086) (width 0.6) (layer "B.Cu") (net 7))
 (segment (start 143.235893 89.834128) (end 144.566457 91.164692) (width 0.6) (layer "B.Cu") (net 7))
 (segment (start 135.445923 80.044247) (end 135.453294 80.036876) (width 0.6) (layer "B.Cu") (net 7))
 (segment (start 142.563448 89.834128) (end 143.235893 89.834128) (width 0.6) (layer "B.Cu") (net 7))
 (segment (start 137.16 53.34) (end 137.16 55.88) (width 0.6) (layer "F.Cu") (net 9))
 (segment (start 127 43.18) (end 137.16 53.34) (width 0.6) (layer "F.Cu") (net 9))
 (segment (start 139.7 78.74) (end 139.68 78.76) (width 0.6) (layer "F.Cu") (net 9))
 (segment (start 137.16 55.88) (end 139.7 58.42) (width 0.6) (layer "F.Cu") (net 9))
 (segment (start 139.7 58.42) (end 139.68 58.44) (width 0.6) (layer "F.Cu") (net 9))
 (segment (start 139.68 58.44) (end 139.68 78.72) (width 0.6) (layer "F.Cu") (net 9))
 (segment (start 124.46 43.18) (end 127 43.18) (width 0.6) (layer "F.Cu") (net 9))
 (segment (start 139.68 78.72) (end 139.7 78.74) (width 0.6) (layer "F.Cu") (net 9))
 (via (at 139.68 78.72) (size 0.8) (drill 0.4) (layers "F.Cu" "B.Cu") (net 9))
 (segment (start 142.59433 87.263246) (end 142.563448 87.294128) (width 0.6) (layer "B.Cu") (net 9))
 (segment (start 145.528136 88.9) (end 143.963439 87.335303) (width 0.6) (layer "B.Cu") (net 9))
 (segment (start 142.604623 87.335303) (end 142.563448 87.294128) (width 0.6) (layer "B.Cu") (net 9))
 (segment (start 142.563448 87.294128) (end 142.054474 87.294128) (width 0.6) (layer "B.Cu") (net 9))
 (segment (start 139.7 84.43068) (end 139.7 78.74) (width 0.6) (layer "B.Cu") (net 9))
 (segment (start 143.963439 87.335303) (end 142.604623 87.335303) (width 0.6) (layer "B.Cu") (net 9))
 (segment (start 142.563448 87.294128) (end 139.7 84.43068) (width 0.6) (layer "B.Cu") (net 9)))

